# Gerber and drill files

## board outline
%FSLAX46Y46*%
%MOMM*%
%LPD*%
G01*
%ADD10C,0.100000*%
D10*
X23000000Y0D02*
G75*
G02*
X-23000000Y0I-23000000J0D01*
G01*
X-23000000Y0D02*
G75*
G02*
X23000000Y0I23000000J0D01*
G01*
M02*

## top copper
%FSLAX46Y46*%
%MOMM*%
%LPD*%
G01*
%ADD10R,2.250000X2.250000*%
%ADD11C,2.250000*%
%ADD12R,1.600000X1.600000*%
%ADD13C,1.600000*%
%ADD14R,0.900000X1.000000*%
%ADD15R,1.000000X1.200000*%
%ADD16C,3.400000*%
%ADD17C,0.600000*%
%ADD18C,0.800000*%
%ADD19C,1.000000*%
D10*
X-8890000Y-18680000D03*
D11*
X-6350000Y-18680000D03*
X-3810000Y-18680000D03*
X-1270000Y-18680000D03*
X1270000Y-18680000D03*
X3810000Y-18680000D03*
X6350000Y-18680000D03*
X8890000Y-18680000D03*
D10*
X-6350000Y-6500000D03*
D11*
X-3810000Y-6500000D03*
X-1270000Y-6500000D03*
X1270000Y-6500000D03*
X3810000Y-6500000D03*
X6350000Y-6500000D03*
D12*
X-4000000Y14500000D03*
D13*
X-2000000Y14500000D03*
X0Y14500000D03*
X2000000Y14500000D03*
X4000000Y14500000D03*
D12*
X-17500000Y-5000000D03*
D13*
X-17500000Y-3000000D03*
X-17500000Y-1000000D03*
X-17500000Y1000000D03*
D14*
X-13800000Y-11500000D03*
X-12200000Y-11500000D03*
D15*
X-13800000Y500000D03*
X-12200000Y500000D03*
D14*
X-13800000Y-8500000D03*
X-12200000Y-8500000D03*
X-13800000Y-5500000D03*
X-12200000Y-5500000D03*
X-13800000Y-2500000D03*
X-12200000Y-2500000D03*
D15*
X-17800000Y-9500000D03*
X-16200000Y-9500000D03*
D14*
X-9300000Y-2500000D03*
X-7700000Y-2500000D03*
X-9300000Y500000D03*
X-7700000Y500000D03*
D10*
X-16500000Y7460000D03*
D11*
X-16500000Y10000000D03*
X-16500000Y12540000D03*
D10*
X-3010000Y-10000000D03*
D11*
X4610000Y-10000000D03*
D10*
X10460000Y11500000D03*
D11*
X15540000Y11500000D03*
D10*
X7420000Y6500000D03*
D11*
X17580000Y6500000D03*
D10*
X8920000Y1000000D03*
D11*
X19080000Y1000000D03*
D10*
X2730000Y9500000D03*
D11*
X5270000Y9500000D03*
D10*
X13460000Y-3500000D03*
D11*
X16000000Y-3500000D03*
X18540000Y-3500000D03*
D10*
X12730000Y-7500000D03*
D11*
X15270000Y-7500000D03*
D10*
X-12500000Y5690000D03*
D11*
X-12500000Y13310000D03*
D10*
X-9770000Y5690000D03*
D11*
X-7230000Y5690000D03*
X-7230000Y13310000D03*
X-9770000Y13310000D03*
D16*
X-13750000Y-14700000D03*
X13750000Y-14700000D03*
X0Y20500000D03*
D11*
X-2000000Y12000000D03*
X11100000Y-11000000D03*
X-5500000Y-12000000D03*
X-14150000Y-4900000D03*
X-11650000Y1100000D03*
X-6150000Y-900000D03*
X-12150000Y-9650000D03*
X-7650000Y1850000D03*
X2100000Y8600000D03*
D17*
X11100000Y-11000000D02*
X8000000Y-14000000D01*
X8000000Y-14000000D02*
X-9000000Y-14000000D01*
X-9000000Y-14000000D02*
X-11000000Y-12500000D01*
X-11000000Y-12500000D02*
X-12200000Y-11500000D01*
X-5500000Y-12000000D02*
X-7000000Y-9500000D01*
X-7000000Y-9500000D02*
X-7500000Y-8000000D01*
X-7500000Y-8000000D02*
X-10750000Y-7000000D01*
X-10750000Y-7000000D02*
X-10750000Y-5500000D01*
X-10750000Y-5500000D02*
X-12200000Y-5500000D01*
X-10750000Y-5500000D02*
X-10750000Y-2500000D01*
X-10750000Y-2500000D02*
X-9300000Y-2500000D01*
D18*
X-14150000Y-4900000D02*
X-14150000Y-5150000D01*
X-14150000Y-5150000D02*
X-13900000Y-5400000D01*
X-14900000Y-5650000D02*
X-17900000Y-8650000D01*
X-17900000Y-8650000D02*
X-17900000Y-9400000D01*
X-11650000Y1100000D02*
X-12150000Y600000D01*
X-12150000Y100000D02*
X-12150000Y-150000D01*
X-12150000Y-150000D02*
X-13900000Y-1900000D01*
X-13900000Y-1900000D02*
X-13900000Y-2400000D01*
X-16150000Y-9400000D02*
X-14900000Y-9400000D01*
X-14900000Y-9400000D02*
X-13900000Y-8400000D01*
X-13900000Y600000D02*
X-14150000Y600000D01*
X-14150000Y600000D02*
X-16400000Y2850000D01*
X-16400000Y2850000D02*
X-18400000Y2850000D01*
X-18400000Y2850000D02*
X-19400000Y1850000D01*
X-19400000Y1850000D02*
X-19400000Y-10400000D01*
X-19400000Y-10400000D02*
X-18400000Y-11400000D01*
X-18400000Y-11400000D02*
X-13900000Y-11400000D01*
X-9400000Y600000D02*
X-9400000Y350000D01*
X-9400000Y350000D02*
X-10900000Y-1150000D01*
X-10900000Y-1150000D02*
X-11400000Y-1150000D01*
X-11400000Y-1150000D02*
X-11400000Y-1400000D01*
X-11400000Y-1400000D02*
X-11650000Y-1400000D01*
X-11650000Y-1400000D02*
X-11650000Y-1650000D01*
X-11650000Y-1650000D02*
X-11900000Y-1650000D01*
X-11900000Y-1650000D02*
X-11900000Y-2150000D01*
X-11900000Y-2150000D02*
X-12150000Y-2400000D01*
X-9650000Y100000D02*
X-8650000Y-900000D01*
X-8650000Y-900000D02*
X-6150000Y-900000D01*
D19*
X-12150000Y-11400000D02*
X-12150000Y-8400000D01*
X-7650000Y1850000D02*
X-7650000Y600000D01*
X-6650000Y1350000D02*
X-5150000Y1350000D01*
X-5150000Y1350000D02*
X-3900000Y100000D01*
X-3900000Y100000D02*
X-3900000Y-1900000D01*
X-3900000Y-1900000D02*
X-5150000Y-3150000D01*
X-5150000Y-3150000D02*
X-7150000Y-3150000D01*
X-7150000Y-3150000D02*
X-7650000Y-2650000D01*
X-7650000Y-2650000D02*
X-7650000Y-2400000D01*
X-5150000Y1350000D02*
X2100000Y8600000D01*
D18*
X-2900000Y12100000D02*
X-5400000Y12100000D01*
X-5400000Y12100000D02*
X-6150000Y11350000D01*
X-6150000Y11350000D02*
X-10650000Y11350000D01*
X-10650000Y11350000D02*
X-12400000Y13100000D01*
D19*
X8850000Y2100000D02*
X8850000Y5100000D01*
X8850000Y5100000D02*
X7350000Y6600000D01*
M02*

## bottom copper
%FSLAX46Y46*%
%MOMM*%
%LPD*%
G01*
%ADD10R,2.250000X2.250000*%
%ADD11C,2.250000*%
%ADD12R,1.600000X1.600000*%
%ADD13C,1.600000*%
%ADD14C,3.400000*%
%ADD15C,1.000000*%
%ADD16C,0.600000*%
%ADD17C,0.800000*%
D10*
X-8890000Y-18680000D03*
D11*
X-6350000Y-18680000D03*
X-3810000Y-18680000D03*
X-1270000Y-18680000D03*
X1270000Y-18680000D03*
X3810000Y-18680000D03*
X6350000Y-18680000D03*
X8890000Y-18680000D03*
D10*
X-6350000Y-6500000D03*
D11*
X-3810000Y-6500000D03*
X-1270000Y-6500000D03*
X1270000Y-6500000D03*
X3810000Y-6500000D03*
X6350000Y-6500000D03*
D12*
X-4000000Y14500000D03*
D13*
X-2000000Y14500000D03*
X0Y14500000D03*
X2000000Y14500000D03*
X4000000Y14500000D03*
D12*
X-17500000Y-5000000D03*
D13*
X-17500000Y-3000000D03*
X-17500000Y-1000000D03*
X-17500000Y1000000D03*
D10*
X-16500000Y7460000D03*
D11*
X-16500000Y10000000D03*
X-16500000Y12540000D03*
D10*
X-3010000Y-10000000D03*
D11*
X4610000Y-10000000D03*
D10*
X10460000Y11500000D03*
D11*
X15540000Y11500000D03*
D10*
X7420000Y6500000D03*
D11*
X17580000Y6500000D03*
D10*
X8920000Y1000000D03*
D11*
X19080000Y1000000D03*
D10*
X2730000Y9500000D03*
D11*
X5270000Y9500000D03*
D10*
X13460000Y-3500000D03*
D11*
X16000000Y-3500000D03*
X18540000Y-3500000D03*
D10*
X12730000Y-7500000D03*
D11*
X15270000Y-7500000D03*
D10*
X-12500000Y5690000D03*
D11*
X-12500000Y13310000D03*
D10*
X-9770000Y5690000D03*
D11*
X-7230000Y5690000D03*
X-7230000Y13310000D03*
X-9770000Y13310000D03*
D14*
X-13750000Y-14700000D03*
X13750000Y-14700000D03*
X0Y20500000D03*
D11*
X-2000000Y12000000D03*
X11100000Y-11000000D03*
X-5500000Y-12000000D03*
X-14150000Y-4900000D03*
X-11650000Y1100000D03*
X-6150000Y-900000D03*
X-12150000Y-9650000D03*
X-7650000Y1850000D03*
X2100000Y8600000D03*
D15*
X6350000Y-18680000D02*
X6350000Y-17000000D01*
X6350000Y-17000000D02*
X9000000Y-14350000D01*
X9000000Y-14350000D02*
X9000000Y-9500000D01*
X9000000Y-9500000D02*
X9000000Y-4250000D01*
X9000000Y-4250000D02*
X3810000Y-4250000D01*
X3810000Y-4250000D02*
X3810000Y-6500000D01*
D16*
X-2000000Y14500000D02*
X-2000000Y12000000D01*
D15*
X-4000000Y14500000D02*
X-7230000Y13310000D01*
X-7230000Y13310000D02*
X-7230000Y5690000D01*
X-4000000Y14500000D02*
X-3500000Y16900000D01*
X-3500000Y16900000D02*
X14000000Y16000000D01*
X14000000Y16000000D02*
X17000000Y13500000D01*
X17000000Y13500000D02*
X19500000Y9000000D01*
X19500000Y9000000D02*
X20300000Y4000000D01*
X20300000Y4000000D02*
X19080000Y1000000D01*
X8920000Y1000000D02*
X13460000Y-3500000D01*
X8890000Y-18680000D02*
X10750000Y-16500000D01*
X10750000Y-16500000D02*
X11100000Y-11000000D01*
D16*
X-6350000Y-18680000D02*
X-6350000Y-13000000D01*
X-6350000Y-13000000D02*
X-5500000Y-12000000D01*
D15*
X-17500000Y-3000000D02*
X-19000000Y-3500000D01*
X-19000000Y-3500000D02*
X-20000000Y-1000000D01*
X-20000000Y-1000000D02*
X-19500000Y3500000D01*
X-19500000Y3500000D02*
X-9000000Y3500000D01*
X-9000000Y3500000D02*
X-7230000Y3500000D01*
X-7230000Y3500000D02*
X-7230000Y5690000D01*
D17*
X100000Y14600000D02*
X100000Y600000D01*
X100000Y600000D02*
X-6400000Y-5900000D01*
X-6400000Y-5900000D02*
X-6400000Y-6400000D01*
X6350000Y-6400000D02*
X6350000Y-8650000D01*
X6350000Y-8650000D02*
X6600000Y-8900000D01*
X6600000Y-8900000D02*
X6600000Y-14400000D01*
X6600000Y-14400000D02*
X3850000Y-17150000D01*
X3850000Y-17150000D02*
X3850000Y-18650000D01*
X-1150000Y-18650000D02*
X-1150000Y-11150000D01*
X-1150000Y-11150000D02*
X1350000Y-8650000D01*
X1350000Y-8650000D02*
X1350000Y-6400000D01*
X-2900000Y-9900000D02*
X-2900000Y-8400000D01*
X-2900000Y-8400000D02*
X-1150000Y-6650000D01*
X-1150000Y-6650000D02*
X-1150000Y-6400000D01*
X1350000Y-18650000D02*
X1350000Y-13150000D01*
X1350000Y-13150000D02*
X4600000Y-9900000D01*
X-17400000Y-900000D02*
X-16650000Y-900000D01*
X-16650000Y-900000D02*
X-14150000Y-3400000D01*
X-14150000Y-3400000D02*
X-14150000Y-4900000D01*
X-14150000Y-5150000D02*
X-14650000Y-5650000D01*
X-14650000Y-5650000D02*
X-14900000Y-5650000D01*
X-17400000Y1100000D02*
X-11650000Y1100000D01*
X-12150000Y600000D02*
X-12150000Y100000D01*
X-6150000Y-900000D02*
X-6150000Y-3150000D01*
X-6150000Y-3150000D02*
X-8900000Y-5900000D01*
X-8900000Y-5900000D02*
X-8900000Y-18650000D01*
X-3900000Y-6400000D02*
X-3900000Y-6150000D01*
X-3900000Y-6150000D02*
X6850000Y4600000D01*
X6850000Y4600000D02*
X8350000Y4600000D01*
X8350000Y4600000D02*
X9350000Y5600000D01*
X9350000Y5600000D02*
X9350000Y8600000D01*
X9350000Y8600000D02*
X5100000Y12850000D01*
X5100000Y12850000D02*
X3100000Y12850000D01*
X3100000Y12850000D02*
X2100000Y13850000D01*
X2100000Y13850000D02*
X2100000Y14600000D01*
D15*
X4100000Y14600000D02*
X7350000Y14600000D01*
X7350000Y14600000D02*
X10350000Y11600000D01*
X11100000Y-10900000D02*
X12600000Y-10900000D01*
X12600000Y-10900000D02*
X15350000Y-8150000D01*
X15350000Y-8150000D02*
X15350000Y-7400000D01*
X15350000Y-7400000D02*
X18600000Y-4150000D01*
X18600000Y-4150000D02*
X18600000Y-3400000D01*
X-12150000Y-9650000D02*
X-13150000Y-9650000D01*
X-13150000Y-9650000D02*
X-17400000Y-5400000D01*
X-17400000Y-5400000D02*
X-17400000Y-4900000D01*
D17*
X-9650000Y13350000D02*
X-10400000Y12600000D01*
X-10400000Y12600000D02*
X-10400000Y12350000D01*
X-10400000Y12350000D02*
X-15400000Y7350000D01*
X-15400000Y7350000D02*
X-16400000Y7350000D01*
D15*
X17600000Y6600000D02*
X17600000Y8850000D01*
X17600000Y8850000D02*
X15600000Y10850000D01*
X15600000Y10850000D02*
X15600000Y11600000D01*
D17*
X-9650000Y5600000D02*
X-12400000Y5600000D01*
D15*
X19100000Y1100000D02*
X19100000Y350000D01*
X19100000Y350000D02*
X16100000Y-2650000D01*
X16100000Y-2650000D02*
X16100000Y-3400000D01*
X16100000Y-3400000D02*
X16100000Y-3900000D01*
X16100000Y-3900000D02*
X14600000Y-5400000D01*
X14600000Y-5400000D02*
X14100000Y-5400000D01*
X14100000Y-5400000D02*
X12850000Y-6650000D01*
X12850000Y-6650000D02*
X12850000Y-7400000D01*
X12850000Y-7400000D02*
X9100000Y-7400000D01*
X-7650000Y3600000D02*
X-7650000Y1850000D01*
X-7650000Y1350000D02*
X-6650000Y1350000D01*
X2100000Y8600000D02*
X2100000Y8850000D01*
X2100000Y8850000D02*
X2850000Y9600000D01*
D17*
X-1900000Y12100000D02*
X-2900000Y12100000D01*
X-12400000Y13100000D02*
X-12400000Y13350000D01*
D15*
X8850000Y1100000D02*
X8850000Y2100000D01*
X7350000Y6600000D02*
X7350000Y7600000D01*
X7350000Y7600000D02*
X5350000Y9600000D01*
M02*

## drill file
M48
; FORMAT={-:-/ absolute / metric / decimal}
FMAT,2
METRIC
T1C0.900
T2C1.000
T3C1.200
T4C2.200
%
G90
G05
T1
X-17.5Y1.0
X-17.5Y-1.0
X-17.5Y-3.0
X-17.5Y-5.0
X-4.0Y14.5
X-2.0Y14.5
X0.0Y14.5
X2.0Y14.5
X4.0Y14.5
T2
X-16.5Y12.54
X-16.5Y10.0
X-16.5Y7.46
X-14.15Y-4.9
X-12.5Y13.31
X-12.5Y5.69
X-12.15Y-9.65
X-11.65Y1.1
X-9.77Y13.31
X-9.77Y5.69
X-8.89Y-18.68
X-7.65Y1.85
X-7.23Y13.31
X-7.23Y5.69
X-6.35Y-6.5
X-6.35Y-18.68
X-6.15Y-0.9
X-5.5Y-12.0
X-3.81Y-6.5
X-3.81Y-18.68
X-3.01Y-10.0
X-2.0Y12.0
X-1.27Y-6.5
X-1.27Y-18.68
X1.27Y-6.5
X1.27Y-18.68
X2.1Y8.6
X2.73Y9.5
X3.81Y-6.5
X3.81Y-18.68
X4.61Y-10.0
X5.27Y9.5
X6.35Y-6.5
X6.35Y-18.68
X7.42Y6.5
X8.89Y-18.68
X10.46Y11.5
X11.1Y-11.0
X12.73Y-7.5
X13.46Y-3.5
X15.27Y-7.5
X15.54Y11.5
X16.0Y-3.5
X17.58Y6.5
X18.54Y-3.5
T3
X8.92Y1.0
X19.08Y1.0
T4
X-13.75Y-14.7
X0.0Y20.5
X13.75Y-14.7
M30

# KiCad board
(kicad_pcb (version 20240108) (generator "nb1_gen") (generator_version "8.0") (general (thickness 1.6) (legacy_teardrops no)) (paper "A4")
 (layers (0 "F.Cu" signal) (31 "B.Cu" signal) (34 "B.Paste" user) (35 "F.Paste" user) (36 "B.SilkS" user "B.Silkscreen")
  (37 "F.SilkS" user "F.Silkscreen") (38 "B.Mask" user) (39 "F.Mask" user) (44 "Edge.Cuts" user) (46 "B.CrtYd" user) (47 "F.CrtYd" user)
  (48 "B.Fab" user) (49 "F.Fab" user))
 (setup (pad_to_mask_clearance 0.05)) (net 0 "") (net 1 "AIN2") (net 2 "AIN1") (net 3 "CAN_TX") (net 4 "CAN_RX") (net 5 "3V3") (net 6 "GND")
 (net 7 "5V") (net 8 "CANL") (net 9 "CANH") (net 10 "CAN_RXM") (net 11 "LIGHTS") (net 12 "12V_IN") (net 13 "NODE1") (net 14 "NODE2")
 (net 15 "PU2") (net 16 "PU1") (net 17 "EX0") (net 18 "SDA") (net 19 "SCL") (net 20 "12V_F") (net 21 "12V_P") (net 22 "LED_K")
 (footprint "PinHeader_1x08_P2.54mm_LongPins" (layer "F.Cu") (at 0 18.68 0)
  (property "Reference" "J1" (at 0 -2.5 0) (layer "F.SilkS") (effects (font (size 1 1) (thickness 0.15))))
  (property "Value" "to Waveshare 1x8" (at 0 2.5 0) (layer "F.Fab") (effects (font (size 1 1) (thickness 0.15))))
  (pad "1" thru_hole rect (at -8.89 0 0) (size 2.25 2.25) (drill 1.0) (layers "*.Cu" "*.Mask") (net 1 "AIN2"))
  (pad "2" thru_hole circle (at -6.35 0 0) (size 2.25 2.25) (drill 1.0) (layers "*.Cu" "*.Mask") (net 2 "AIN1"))
  (pad "3" thru_hole circle (at -3.81 0 0) (size 2.25 2.25) (drill 1.0) (layers "*.Cu" "*.Mask"))
  (pad "4" thru_hole circle (at -1.27 0 0) (size 2.25 2.25) (drill 1.0) (layers "*.Cu" "*.Mask") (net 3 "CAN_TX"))
  (pad "5" thru_hole circle (at 1.27 0 0) (size 2.25 2.25) (drill 1.0) (layers "*.Cu" "*.Mask") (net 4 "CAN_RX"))
  (pad "6" thru_hole circle (at 3.81 0 0) (size 2.25 2.25) (drill 1.0) (layers "*.Cu" "*.Mask") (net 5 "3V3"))
  (pad "7" thru_hole circle (at 6.35 0 0) (size 2.25 2.25) (drill 1.0) (layers "*.Cu" "*.Mask") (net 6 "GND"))
  (pad "8" thru_hole circle (at 8.89 0 0) (size 2.25 2.25) (drill 1.0) (layers "*.Cu" "*.Mask") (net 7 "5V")))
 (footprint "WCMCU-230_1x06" (layer "F.Cu") (at 0 6.5 0)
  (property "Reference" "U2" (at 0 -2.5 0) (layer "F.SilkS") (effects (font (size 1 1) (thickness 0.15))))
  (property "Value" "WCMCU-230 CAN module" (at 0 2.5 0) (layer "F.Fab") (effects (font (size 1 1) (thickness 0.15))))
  (pad "1" thru_hole rect (at -6.35 0 0) (size 2.25 2.25) (drill 1.0) (layers "*.Cu" "*.Mask") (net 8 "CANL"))
  (pad "2" thru_hole circle (at -3.81 0 0) (size 2.25 2.25) (drill 1.0) (layers "*.Cu" "*.Mask") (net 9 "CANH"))
  (pad "3" thru_hole circle (at -1.27 0 0) (size 2.25 2.25) (drill 1.0) (layers "*.Cu" "*.Mask") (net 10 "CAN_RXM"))
  (pad "4" thru_hole circle (at 1.27 0 0) (size 2.25 2.25) (drill 1.0) (layers "*.Cu" "*.Mask") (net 3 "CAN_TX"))
  (pad "5" thru_hole circle (at 3.81 0 0) (size 2.25 2.25) (drill 1.0) (layers "*.Cu" "*.Mask") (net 6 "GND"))
  (pad "6" thru_hole circle (at 6.35 0 0) (size 2.25 2.25) (drill 1.0) (layers "*.Cu" "*.Mask") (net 5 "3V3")))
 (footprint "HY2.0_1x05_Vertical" (layer "F.Cu") (at 0 -14.5 0)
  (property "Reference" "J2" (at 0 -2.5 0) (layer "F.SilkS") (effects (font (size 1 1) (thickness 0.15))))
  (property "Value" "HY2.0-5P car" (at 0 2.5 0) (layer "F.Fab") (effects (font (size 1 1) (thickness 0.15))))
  (pad "1" thru_hole rect (at -4.0 0 0) (size 1.6 1.6) (drill 0.9) (layers "*.Cu" "*.Mask") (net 6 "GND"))
  (pad "2" thru_hole circle (at -2.0 0 0) (size 1.6 1.6) (drill 0.9) (layers "*.Cu" "*.Mask") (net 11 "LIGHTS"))
  (pad "3" thru_hole circle (at 0.0 0 0) (size 1.6 1.6) (drill 0.9) (layers "*.Cu" "*.Mask") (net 8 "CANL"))
  (pad "4" thru_hole circle (at 2.0 0 0) (size 1.6 1.6) (drill 0.9) (layers "*.Cu" "*.Mask") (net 9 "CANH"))
  (pad "5" thru_hole circle (at 4.0 0 0) (size 1.6 1.6) (drill 0.9) (layers "*.Cu" "*.Mask") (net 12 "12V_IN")))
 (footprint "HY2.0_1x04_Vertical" (layer "F.Cu") (at -17.5 2.0 0)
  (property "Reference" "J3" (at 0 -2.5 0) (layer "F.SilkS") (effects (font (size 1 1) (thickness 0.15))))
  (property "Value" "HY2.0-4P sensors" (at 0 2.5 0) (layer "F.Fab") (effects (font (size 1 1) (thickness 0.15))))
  (pad "1" thru_hole rect (at 0 3.0 0) (size 1.6 1.6) (drill 0.9) (layers "*.Cu" "*.Mask") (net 7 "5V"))
  (pad "2" thru_hole circle (at 0 1.0 0) (size 1.6 1.6) (drill 0.9) (layers "*.Cu" "*.Mask") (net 6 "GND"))
  (pad "3" thru_hole circle (at 0 -1.0 0) (size 1.6 1.6) (drill 0.9) (layers "*.Cu" "*.Mask") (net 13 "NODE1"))
  (pad "4" thru_hole circle (at 0 -3.0 0) (size 1.6 1.6) (drill 0.9) (layers "*.Cu" "*.Mask") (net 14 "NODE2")))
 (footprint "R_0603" (layer "F.Cu") (at -13.0 11.5 0)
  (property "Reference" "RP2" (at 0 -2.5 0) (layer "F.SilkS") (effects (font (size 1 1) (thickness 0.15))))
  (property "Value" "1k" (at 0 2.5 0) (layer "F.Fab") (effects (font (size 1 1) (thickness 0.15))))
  (pad "1" smd rect (at -0.8 0 0) (size 0.9 1.0) (layers "F.Cu" "F.Mask") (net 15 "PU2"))
  (pad "2" smd rect (at 0.8 0 0) (size 0.9 1.0) (layers "F.Cu" "F.Mask") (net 7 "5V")))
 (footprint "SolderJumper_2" (layer "F.Cu") (at -13.0 -0.5 0)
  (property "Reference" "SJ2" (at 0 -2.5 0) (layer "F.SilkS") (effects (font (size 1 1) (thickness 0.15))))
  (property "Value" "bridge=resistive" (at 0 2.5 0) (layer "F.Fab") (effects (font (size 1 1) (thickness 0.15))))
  (pad "1" smd rect (at -0.8 0 0) (size 1.0 1.2) (layers "F.Cu" "F.Mask") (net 15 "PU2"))
  (pad "2" smd rect (at 0.8 0 0) (size 1.0 1.2) (layers "F.Cu" "F.Mask") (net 14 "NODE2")))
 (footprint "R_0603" (layer "F.Cu") (at -13.0 8.5 0)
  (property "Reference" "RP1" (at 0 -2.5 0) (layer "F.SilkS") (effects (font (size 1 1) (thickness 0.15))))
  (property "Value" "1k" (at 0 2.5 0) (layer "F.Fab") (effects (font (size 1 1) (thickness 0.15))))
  (pad "1" smd rect (at -0.8 0 0) (size 0.9 1.0) (layers "F.Cu" "F.Mask") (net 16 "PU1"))
  (pad "2" smd rect (at 0.8 0 0) (size 0.9 1.0) (layers "F.Cu" "F.Mask") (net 7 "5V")))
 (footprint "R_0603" (layer "F.Cu") (at -13.0 5.5 0)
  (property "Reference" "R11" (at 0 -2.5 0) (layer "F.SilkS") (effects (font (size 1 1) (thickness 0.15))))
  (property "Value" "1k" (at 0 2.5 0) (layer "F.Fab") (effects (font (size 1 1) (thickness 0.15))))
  (pad "1" smd rect (at -0.8 0 0) (size 0.9 1.0) (layers "F.Cu" "F.Mask") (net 13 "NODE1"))
  (pad "2" smd rect (at 0.8 0 0) (size 0.9 1.0) (layers "F.Cu" "F.Mask") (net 2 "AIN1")))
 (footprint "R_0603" (layer "F.Cu") (at -13.0 2.5 0)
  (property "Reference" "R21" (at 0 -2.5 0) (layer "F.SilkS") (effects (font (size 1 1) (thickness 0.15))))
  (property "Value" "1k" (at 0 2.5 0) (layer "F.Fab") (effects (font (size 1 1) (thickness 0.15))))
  (pad "1" smd rect (at -0.8 0 0) (size 0.9 1.0) (layers "F.Cu" "F.Mask") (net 14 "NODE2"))
  (pad "2" smd rect (at 0.8 0 0) (size 0.9 1.0) (layers "F.Cu" "F.Mask") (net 1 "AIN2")))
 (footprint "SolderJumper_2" (layer "F.Cu") (at -17.0 9.5 0)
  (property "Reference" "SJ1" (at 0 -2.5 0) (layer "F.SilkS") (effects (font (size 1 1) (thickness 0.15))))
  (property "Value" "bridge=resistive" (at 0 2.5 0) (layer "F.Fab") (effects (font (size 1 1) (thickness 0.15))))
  (pad "1" smd rect (at -0.8 0 0) (size 1.0 1.2) (layers "F.Cu" "F.Mask") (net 13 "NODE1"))
  (pad "2" smd rect (at 0.8 0 0) (size 1.0 1.2) (layers "F.Cu" "F.Mask") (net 16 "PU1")))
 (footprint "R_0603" (layer "F.Cu") (at -8.5 2.5 0)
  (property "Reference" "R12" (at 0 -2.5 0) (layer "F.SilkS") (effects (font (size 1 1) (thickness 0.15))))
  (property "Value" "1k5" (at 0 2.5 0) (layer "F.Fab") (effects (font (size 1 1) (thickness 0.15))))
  (pad "1" smd rect (at -0.8 0 0) (size 0.9 1.0) (layers "F.Cu" "F.Mask") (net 2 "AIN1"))
  (pad "2" smd rect (at 0.8 0 0) (size 0.9 1.0) (layers "F.Cu" "F.Mask") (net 6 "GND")))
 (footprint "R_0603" (layer "F.Cu") (at -8.5 -0.5 0)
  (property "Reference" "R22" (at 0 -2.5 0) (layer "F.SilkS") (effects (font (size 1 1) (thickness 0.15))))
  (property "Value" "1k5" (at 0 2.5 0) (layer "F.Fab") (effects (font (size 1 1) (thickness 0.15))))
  (pad "1" smd rect (at -0.8 0 0) (size 0.9 1.0) (layers "F.Cu" "F.Mask") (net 1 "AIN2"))
  (pad "2" smd rect (at 0.8 0 0) (size 0.9 1.0) (layers "F.Cu" "F.Mask") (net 6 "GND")))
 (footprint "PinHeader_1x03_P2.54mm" (layer "F.Cu") (at -16.5 -10.0 0)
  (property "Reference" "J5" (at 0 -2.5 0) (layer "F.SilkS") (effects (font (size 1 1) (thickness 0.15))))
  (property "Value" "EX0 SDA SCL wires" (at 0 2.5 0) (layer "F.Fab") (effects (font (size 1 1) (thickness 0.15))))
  (pad "1" thru_hole rect (at 0 2.54 0) (size 2.25 2.25) (drill 1.0) (layers "*.Cu" "*.Mask") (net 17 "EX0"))
  (pad "2" thru_hole circle (at 0 -0.0 0) (size 2.25 2.25) (drill 1.0) (layers "*.Cu" "*.Mask") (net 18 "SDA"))
  (pad "3" thru_hole circle (at 0 -2.54 0) (size 2.25 2.25) (drill 1.0) (layers "*.Cu" "*.Mask") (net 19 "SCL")))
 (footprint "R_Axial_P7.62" (layer "F.Cu") (at 0.8 10.0 0)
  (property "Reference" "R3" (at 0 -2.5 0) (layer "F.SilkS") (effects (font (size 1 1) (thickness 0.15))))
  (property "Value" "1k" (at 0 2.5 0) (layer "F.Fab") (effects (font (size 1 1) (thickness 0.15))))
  (pad "1" thru_hole rect (at -3.81 0 0) (size 2.25 2.25) (drill 1.0) (layers "*.Cu" "*.Mask") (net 10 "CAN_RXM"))
  (pad "2" thru_hole circle (at 3.81 0 0) (size 2.25 2.25) (drill 1.0) (layers "*.Cu" "*.Mask") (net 4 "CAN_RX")))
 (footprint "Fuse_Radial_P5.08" (layer "F.Cu") (at 13.0 -11.5 0)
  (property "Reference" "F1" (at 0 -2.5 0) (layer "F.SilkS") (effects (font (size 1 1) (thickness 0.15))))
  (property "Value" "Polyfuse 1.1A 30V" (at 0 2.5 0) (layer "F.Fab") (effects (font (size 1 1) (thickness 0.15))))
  (pad "1" thru_hole rect (at -2.54 0 0) (size 2.25 2.25) (drill 1.0) (layers "*.Cu" "*.Mask") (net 12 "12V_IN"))
  (pad "2" thru_hole circle (at 2.54 0 0) (size 2.25 2.25) (drill 1.0) (layers "*.Cu" "*.Mask") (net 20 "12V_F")))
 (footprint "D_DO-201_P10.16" (layer "F.Cu") (at 12.5 -6.5 0)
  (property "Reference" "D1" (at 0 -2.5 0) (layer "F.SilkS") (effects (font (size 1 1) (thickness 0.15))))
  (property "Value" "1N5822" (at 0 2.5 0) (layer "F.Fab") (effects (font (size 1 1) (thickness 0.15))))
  (pad "1" thru_hole rect (at -5.08 0 0) (size 2.25 2.25) (drill 1.0) (layers "*.Cu" "*.Mask") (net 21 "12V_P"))
  (pad "2" thru_hole circle (at 5.08 0 0) (size 2.25 2.25) (drill 1.0) (layers "*.Cu" "*.Mask") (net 20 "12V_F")))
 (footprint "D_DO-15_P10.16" (layer "F.Cu") (at 14.0 -1.0 0)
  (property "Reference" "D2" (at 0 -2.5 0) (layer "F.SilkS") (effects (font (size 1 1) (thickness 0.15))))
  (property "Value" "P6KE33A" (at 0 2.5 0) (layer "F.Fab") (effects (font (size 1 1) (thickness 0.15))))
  (pad "1" thru_hole rect (at -5.08 0 0) (size 2.25 2.25) (drill 1.2) (layers "*.Cu" "*.Mask") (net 21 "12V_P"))
  (pad "2" thru_hole circle (at 5.08 0 0) (size 2.25 2.25) (drill 1.2) (layers "*.Cu" "*.Mask") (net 6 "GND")))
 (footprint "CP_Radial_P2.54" (layer "F.Cu") (at 4.0 -9.5 0)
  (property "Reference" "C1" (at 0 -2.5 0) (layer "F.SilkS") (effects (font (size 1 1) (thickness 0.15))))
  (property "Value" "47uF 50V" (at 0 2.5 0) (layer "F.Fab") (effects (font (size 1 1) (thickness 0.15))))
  (pad "1" thru_hole rect (at -1.27 0 0) (size 2.25 2.25) (drill 1.0) (layers "*.Cu" "*.Mask") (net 6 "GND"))
  (pad "2" thru_hole circle (at 1.27 0 0) (size 2.25 2.25) (drill 1.0) (layers "*.Cu" "*.Mask") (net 21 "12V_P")))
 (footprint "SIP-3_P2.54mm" (layer "F.Cu") (at 16.0 3.5 0)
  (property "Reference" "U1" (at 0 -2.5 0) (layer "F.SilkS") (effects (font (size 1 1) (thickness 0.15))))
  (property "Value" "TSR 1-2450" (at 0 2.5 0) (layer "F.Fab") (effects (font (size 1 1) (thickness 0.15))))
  (pad "1" thru_hole rect (at -2.54 0 0) (size 2.25 2.25) (drill 1.0) (layers "*.Cu" "*.Mask") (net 21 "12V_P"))
  (pad "2" thru_hole circle (at 0.0 0 0) (size 2.25 2.25) (drill 1.0) (layers "*.Cu" "*.Mask") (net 6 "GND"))
  (pad "3" thru_hole circle (at 2.54 0 0) (size 2.25 2.25) (drill 1.0) (layers "*.Cu" "*.Mask") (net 7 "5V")))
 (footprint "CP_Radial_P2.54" (layer "F.Cu") (at 14.0 7.5 0)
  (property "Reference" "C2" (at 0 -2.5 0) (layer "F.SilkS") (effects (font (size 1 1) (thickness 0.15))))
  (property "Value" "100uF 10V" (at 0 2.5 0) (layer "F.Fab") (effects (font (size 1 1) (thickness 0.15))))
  (pad "1" thru_hole rect (at -1.27 0 0) (size 2.25 2.25) (drill 1.0) (layers "*.Cu" "*.Mask") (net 6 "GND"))
  (pad "2" thru_hole circle (at 1.27 0 0) (size 2.25 2.25) (drill 1.0) (layers "*.Cu" "*.Mask") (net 7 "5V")))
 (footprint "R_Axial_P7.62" (layer "F.Cu") (at -12.5 -9.5 90)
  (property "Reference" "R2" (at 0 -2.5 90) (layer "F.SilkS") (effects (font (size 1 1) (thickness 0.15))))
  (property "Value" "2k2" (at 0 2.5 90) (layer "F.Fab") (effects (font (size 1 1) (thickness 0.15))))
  (pad "1" thru_hole rect (at -3.81 0 90) (size 2.25 2.25) (drill 1.0) (layers "*.Cu" "*.Mask") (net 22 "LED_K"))
  (pad "2" thru_hole circle (at 3.81 0 90) (size 2.25 2.25) (drill 1.0) (layers "*.Cu" "*.Mask") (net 11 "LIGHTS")))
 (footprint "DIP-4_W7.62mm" (layer "F.Cu") (at -8.5 -9.5 0)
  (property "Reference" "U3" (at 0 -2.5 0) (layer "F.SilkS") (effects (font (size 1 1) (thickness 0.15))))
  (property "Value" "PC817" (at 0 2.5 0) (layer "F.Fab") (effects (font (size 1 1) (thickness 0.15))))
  (pad "1" thru_hole rect (at -1.27 3.81 0) (size 2.25 2.25) (drill 1.0) (layers "*.Cu" "*.Mask") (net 22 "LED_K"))
  (pad "2" thru_hole circle (at 1.27 3.81 0) (size 2.25 2.25) (drill 1.0) (layers "*.Cu" "*.Mask") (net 6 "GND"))
  (pad "3" thru_hole circle (at 1.27 -3.81 0) (size 2.25 2.25) (drill 1.0) (layers "*.Cu" "*.Mask") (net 6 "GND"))
  (pad "4" thru_hole circle (at -1.27 -3.81 0) (size 2.25 2.25) (drill 1.0) (layers "*.Cu" "*.Mask") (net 17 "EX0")))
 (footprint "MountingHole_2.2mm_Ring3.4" (layer "F.Cu") (at -13.75 14.7 0)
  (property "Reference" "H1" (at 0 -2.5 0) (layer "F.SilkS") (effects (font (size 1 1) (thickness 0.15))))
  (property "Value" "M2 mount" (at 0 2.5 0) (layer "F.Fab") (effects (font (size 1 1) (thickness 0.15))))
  (pad "1" thru_hole circle (at 0 0 0) (size 3.4 3.4) (drill 2.2) (layers "*.Cu" "*.Mask")))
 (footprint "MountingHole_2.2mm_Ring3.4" (layer "F.Cu") (at 13.75 14.7 0)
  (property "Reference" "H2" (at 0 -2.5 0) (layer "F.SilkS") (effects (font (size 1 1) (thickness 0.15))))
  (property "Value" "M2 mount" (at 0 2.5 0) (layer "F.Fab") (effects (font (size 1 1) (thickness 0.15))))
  (pad "1" thru_hole circle (at 0 0 0) (size 3.4 3.4) (drill 2.2) (layers "*.Cu" "*.Mask")))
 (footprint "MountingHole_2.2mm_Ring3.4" (layer "F.Cu") (at 0 -20.5 0)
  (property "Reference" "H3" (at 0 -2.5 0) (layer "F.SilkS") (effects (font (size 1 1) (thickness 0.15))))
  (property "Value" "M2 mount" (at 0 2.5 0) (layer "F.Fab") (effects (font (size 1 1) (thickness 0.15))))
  (pad "1" thru_hole circle (at 0 0 0) (size 3.4 3.4) (drill 2.2) (layers "*.Cu" "*.Mask")))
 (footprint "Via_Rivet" (layer "F.Cu") (at -2.0 -12.0 0)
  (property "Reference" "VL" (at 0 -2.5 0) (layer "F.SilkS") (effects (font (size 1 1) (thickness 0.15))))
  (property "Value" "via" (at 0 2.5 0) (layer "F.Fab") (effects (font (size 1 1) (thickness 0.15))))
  (pad "1" thru_hole circle (at 0 0 0) (size 2.25 2.25) (drill 1.0) (layers "*.Cu" "*.Mask") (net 11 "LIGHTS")))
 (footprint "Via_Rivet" (layer "F.Cu") (at 11.1 11.0 0)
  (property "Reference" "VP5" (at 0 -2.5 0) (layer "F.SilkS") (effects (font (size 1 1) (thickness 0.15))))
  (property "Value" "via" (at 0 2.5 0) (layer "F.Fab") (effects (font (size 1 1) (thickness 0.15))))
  (pad "1" thru_hole circle (at 0 0 0) (size 2.25 2.25) (drill 1.0) (layers "*.Cu" "*.Mask") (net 7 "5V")))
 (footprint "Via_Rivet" (layer "F.Cu") (at -5.5 12.0 0)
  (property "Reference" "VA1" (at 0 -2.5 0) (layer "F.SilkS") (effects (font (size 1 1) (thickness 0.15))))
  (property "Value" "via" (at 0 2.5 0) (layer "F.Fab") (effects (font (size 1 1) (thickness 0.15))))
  (pad "1" thru_hole circle (at 0 0 0) (size 2.25 2.25) (drill 1.0) (layers "*.Cu" "*.Mask") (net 2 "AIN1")))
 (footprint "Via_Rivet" (layer "F.Cu") (at -14.15 4.9 0)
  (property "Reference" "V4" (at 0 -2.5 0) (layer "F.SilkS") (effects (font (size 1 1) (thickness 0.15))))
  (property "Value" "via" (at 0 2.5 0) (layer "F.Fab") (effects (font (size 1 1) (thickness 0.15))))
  (pad "1" thru_hole circle (at 0 0 0) (size 2.25 2.25) (drill 1.0) (layers "*.Cu" "*.Mask") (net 13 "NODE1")))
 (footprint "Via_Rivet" (layer "F.Cu") (at -11.65 -1.1 0)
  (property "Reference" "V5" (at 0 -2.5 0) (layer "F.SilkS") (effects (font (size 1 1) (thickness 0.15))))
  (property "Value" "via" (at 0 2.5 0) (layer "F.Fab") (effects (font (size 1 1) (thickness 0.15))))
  (pad "1" thru_hole circle (at 0 0 0) (size 2.25 2.25) (drill 1.0) (layers "*.Cu" "*.Mask") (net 14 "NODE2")))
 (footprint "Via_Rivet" (layer "F.Cu") (at -6.15 0.9 0)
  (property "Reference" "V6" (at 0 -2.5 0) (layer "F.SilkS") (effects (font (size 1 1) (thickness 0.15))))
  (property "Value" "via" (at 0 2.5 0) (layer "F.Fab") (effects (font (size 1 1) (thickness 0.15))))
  (pad "1" thru_hole circle (at 0 0 0) (size 2.25 2.25) (drill 1.0) (layers "*.Cu" "*.Mask") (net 1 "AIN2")))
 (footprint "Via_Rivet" (layer "F.Cu") (at -12.15 9.65 0)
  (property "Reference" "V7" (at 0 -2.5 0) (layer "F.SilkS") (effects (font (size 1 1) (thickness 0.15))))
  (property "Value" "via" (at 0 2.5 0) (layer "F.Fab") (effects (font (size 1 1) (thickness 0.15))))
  (pad "1" thru_hole circle (at 0 0 0) (size 2.25 2.25) (drill 1.0) (layers "*.Cu" "*.Mask") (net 7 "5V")))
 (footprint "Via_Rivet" (layer "F.Cu") (at -7.65 -1.85 0)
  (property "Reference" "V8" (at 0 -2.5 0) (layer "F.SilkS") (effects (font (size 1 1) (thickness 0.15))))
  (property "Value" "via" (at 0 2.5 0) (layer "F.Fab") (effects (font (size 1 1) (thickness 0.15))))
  (pad "1" thru_hole circle (at 0 0 0) (size 2.25 2.25) (drill 1.0) (layers "*.Cu" "*.Mask") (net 6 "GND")))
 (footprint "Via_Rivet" (layer "F.Cu") (at 2.1 -8.6 0)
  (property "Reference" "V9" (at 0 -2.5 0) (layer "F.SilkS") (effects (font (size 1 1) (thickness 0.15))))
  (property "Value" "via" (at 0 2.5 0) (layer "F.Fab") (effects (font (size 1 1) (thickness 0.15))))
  (pad "1" thru_hole circle (at 0 0 0) (size 2.25 2.25) (drill 1.0) (layers "*.Cu" "*.Mask") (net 6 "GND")))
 (gr_circle (center 0 0) (end 23.0 0) (stroke (width 0.1) (type default)) (fill none) (layer "Edge.Cuts"))
 (segment (start 6.35 18.68) (end 6.35 17.0) (width 1.0) (layer "B.Cu") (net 6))
 (segment (start 6.35 17.0) (end 9.0 14.35) (width 1.0) (layer "B.Cu") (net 6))
 (segment (start 9.0 14.35) (end 9.0 9.5) (width 1.0) (layer "B.Cu") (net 6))
 (segment (start 9.0 9.5) (end 9.0 4.25) (width 1.0) (layer "B.Cu") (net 6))
 (segment (start 9.0 4.25) (end 3.81 4.25) (width 1.0) (layer "B.Cu") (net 6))
 (segment (start 3.81 4.25) (end 3.81 6.5) (width 1.0) (layer "B.Cu") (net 6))
 (segment (start -2.0 -14.5) (end -2.0 -12.0) (width 0.6) (layer "B.Cu") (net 11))
 (segment (start -4.0 -14.5) (end -7.23 -13.31) (width 1.0) (layer "B.Cu") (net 6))
 (segment (start -7.23 -13.31) (end -7.23 -5.69) (width 1.0) (layer "B.Cu") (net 6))
 (segment (start -4.0 -14.5) (end -3.5 -16.9) (width 1.0) (layer "B.Cu") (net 6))
 (segment (start -3.5 -16.9) (end 14.0 -16.0) (width 1.0) (layer "B.Cu") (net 6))
 (segment (start 14.0 -16.0) (end 17.0 -13.5) (width 1.0) (layer "B.Cu") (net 6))
 (segment (start 17.0 -13.5) (end 19.5 -9.0) (width 1.0) (layer "B.Cu") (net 6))
 (segment (start 19.5 -9.0) (end 20.3 -4.0) (width 1.0) (layer "B.Cu") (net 6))
 (segment (start 20.3 -4.0) (end 19.08 -1.0) (width 1.0) (layer "B.Cu") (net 6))
 (segment (start 8.92 -1.0) (end 13.46 3.5) (width 1.0) (layer "B.Cu") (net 21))
 (segment (start 8.89 18.68) (end 10.75 16.5) (width 1.0) (layer "B.Cu") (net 7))
 (segment (start 10.75 16.5) (end 11.1 11.0) (width 1.0) (layer "B.Cu") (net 7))
 (segment (start 11.1 11.0) (end 8.0 14.0) (width 0.6) (layer "F.Cu") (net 7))
 (segment (start 8.0 14.0) (end -9.0 14.0) (width 0.6) (layer "F.Cu") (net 7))
 (segment (start -9.0 14.0) (end -11.0 12.5) (width 0.6) (layer "F.Cu") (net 7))
 (segment (start -11.0 12.5) (end -12.2 11.5) (width 0.6) (layer "F.Cu") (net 7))
 (segment (start -6.35 18.68) (end -6.35 13.0) (width 0.6) (layer "B.Cu") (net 2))
 (segment (start -6.35 13.0) (end -5.5 12.0) (width 0.6) (layer "B.Cu") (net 2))
 (segment (start -5.5 12.0) (end -7.0 9.5) (width 0.6) (layer "F.Cu") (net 2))
 (segment (start -7.0 9.5) (end -7.5 8.0) (width 0.6) (layer "F.Cu") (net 2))
 (segment (start -7.5 8.0) (end -10.75 7.0) (width 0.6) (layer "F.Cu") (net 2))
 (segment (start -10.75 7.0) (end -10.75 5.5) (width 0.6) (layer "F.Cu") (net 2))
 (segment (start -10.75 5.5) (end -12.2 5.5) (width 0.6) (layer "F.Cu") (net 2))
 (segment (start -10.75 5.5) (end -10.75 2.5) (width 0.6) (layer "F.Cu") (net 2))
 (segment (start -10.75 2.5) (end -9.3 2.5) (width 0.6) (layer "F.Cu") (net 2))
 (segment (start -17.5 3.0) (end -19.0 3.5) (width 1.0) (layer "B.Cu") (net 6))
 (segment (start -19.0 3.5) (end -20.0 1.0) (width 1.0) (layer "B.Cu") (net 6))
 (segment (start -20.0 1.0) (end -19.5 -3.5) (width 1.0) (layer "B.Cu") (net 6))
 (segment (start -19.5 -3.5) (end -9.0 -3.5) (width 1.0) (layer "B.Cu") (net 6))
 (segment (start -9.0 -3.5) (end -7.23 -3.5) (width 1.0) (layer "B.Cu") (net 6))
 (segment (start -7.23 -3.5) (end -7.23 -5.69) (width 1.0) (layer "B.Cu") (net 6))
 (segment (start 0.1 -14.6) (end 0.1 -0.6) (width 0.8) (layer "B.Cu") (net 8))
 (segment (start 0.1 -0.6) (end -6.4 5.9) (width 0.8) (layer "B.Cu") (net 8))
 (segment (start -6.4 5.9) (end -6.4 6.4) (width 0.8) (layer "B.Cu") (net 8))
 (segment (start 6.35 6.4) (end 6.35 8.65) (width 0.8) (layer "B.Cu") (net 5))
 (segment (start 6.35 8.65) (end 6.6 8.9) (width 0.8) (layer "B.Cu") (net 5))
 (segment (start 6.6 8.9) (end 6.6 14.4) (width 0.8) (layer "B.Cu") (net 5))
 (segment (start 6.6 14.4) (end 3.85 17.15) (width 0.8) (layer "B.Cu") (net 5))
 (segment (start 3.85 17.15) (end 3.85 18.65) (width 0.8) (layer "B.Cu") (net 5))
 (segment (start -1.15 18.65) (end -1.15 11.15) (width 0.8) (layer "B.Cu") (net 3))
 (segment (start -1.15 11.15) (end 1.35 8.65) (width 0.8) (layer "B.Cu") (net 3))
 (segment (start 1.35 8.65) (end 1.35 6.4) (width 0.8) (layer "B.Cu") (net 3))
 (segment (start -2.9 9.9) (end -2.9 8.4) (width 0.8) (layer "B.Cu") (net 10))
 (segment (start -2.9 8.4) (end -1.15 6.65) (width 0.8) (layer "B.Cu") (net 10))
 (segment (start -1.15 6.65) (end -1.15 6.4) (width 0.8) (layer "B.Cu") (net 10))
 (segment (start 1.35 18.65) (end 1.35 13.15) (width 0.8) (layer "B.Cu") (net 4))
 (segment (start 1.35 13.15) (end 4.6 9.9) (width 0.8) (layer "B.Cu") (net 4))
 (segment (start -17.4 0.9) (end -16.65 0.9) (width 0.8) (layer "B.Cu") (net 13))
 (segment (start -16.65 0.9) (end -14.15 3.4) (width 0.8) (layer "B.Cu") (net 13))
 (segment (start -14.15 3.4) (end -14.15 4.9) (width 0.8) (layer "B.Cu") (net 13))
 (segment (start -14.15 4.9) (end -14.15 5.15) (width 0.8) (layer "F.Cu") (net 13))
 (segment (start -14.15 5.15) (end -13.9 5.4) (width 0.8) (layer "F.Cu") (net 13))
 (segment (start -14.15 5.15) (end -14.65 5.65) (width 0.8) (layer "B.Cu") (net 13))
 (segment (start -14.65 5.65) (end -14.9 5.65) (width 0.8) (layer "B.Cu") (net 13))
 (segment (start -14.9 5.65) (end -17.9 8.65) (width 0.8) (layer "F.Cu") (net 13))
 (segment (start -17.9 8.65) (end -17.9 9.4) (width 0.8) (layer "F.Cu") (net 13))
 (segment (start -17.4 -1.1) (end -11.65 -1.1) (width 0.8) (layer "B.Cu") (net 14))
 (segment (start -11.65 -1.1) (end -12.15 -0.6) (width 0.8) (layer "F.Cu") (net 14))
 (segment (start -12.15 -0.6) (end -12.15 -0.1) (width 0.8) (layer "B.Cu") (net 14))
 (segment (start -12.15 -0.1) (end -12.15 0.15) (width 0.8) (layer "F.Cu") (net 14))
 (segment (start -12.15 0.15) (end -13.9 1.9) (width 0.8) (layer "F.Cu") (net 14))
 (segment (start -13.9 1.9) (end -13.9 2.4) (width 0.8) (layer "F.Cu") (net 14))
 (segment (start -16.15 9.4) (end -14.9 9.4) (width 0.8) (layer "F.Cu") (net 16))
 (segment (start -14.9 9.4) (end -13.9 8.4) (width 0.8) (layer "F.Cu") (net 16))
 (segment (start -13.9 -0.6) (end -14.15 -0.6) (width 0.8) (layer "F.Cu") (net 15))
 (segment (start -14.15 -0.6) (end -16.4 -2.85) (width 0.8) (layer "F.Cu") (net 15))
 (segment (start -16.4 -2.85) (end -18.4 -2.85) (width 0.8) (layer "F.Cu") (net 15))
 (segment (start -18.4 -2.85) (end -19.4 -1.85) (width 0.8) (layer "F.Cu") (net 15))
 (segment (start -19.4 -1.85) (end -19.4 10.4) (width 0.8) (layer "F.Cu") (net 15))
 (segment (start -19.4 10.4) (end -18.4 11.4) (width 0.8) (layer "F.Cu") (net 15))
 (segment (start -18.4 11.4) (end -13.9 11.4) (width 0.8) (layer "F.Cu") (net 15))
 (segment (start -9.4 -0.6) (end -9.4 -0.35) (width 0.8) (layer "F.Cu") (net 1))
 (segment (start -9.4 -0.35) (end -10.9 1.15) (width 0.8) (layer "F.Cu") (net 1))
 (segment (start -10.9 1.15) (end -11.4 1.15) (width 0.8) (layer "F.Cu") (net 1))
 (segment (start -11.4 1.15) (end -11.4 1.4) (width 0.8) (layer "F.Cu") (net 1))
 (segment (start -11.4 1.4) (end -11.65 1.4) (width 0.8) (layer "F.Cu") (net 1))
 (segment (start -11.65 1.4) (end -11.65 1.65) (width 0.8) (layer "F.Cu") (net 1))
 (segment (start -11.65 1.65) (end -11.9 1.65) (width 0.8) (layer "F.Cu") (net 1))
 (segment (start -11.9 1.65) (end -11.9 2.15) (width 0.8) (layer "F.Cu") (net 1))
 (segment (start -11.9 2.15) (end -12.15 2.4) (width 0.8) (layer "F.Cu") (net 1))
 (segment (start -9.65 -0.1) (end -8.65 0.9) (width 0.8) (layer "F.Cu") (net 1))
 (segment (start -8.65 0.9) (end -6.15 0.9) (width 0.8) (layer "F.Cu") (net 1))
 (segment (start -6.15 0.9) (end -6.15 3.15) (width 0.8) (layer "B.Cu") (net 1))
 (segment (start -6.15 3.15) (end -8.9 5.9) (width 0.8) (layer "B.Cu") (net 1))
 (segment (start -8.9 5.9) (end -8.9 18.65) (width 0.8) (layer "B.Cu") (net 1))
 (segment (start -3.9 6.4) (end -3.9 6.15) (width 0.8) (layer "B.Cu") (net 9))
 (segment (start -3.9 6.15) (end 6.85 -4.6) (width 0.8) (layer "B.Cu") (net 9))
 (segment (start 6.85 -4.6) (end 8.35 -4.6) (width 0.8) (layer "B.Cu") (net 9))
 (segment (start 8.35 -4.6) (end 9.35 -5.6) (width 0.8) (layer "B.Cu") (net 9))
 (segment (start 9.35 -5.6) (end 9.35 -8.6) (width 0.8) (layer "B.Cu") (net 9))
 (segment (start 9.35 -8.6) (end 5.1 -12.85) (width 0.8) (layer "B.Cu") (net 9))
 (segment (start 5.1 -12.85) (end 3.1 -12.85) (width 0.8) (layer "B.Cu") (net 9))
 (segment (start 3.1 -12.85) (end 2.1 -13.85) (width 0.8) (layer "B.Cu") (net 9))
 (segment (start 2.1 -13.85) (end 2.1 -14.6) (width 0.8) (layer "B.Cu") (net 9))
 (segment (start 4.1 -14.6) (end 7.35 -14.6) (width 1.0) (layer "B.Cu") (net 12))
 (segment (start 7.35 -14.6) (end 10.35 -11.6) (width 1.0) (layer "B.Cu") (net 12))
 (segment (start -12.15 11.4) (end -12.15 8.4) (width 1.0) (layer "F.Cu") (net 7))
 (segment (start 11.1 10.9) (end 12.6 10.9) (width 1.0) (layer "B.Cu") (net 7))
 (segment (start 12.6 10.9) (end 15.35 8.15) (width 1.0) (layer "B.Cu") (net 7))
 (segment (start 15.35 8.15) (end 15.35 7.4) (width 1.0) (layer "B.Cu") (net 7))
 (segment (start 15.35 7.4) (end 18.6 4.15) (width 1.0) (layer "B.Cu") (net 7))
 (segment (start 18.6 4.15) (end 18.6 3.4) (width 1.0) (layer "B.Cu") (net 7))
 (segment (start -12.15 9.65) (end -13.15 9.65) (width 1.0) (layer "B.Cu") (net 7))
 (segment (start -13.15 9.65) (end -17.4 5.4) (width 1.0) (layer "B.Cu") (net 7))
 (segment (start -17.4 5.4) (end -17.4 4.9) (width 1.0) (layer "B.Cu") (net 7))
 (segment (start -9.65 -13.35) (end -10.4 -12.6) (width 0.8) (layer "B.Cu") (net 17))
 (segment (start -10.4 -12.6) (end -10.4 -12.35) (width 0.8) (layer "B.Cu") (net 17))
 (segment (start -10.4 -12.35) (end -15.4 -7.35) (width 0.8) (layer "B.Cu") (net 17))
 (segment (start -15.4 -7.35) (end -16.4 -7.35) (width 0.8) (layer "B.Cu") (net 17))
 (segment (start 17.6 -6.6) (end 17.6 -8.85) (width 1.0) (layer "B.Cu") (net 20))
 (segment (start 17.6 -8.85) (end 15.6 -10.85) (width 1.0) (layer "B.Cu") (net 20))
 (segment (start 15.6 -10.85) (end 15.6 -11.6) (width 1.0) (layer "B.Cu") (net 20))
 (segment (start -9.65 -5.6) (end -12.4 -5.6) (width 0.8) (layer "B.Cu") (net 22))
 (segment (start 19.1 -1.1) (end 19.1 -0.35) (width 1.0) (layer "B.Cu") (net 6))
 (segment (start 19.1 -0.35) (end 16.1 2.65) (width 1.0) (layer "B.Cu") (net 6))
 (segment (start 16.1 2.65) (end 16.1 3.4) (width 1.0) (layer "B.Cu") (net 6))
 (segment (start 16.1 3.4) (end 16.1 3.9) (width 1.0) (layer "B.Cu") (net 6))
 (segment (start 16.1 3.9) (end 14.6 5.4) (width 1.0) (layer "B.Cu") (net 6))
 (segment (start 14.6 5.4) (end 14.1 5.4) (width 1.0) (layer "B.Cu") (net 6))
 (segment (start 14.1 5.4) (end 12.85 6.65) (width 1.0) (layer "B.Cu") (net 6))
 (segment (start 12.85 6.65) (end 12.85 7.4) (width 1.0) (layer "B.Cu") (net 6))
 (segment (start 12.85 7.4) (end 9.1 7.4) (width 1.0) (layer "B.Cu") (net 6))
 (segment (start -7.65 -3.6) (end -7.65 -1.85) (width 1.0) (layer "B.Cu") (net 6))
 (segment (start -7.65 -1.85) (end -7.65 -0.6) (width 1.0) (layer "F.Cu") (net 6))
 (segment (start -7.65 -1.35) (end -6.65 -1.35) (width 1.0) (layer "B.Cu") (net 6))
 (segment (start -6.65 -1.35) (end -5.15 -1.35) (width 1.0) (layer "F.Cu") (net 6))
 (segment (start -5.15 -1.35) (end -3.9 -0.1) (width 1.0) (layer "F.Cu") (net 6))
 (segment (start -3.9 -0.1) (end -3.9 1.9) (width 1.0) (layer "F.Cu") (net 6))
 (segment (start -3.9 1.9) (end -5.15 3.15) (width 1.0) (layer "F.Cu") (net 6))
 (segment (start -5.15 3.15) (end -7.15 3.15) (width 1.0) (layer "F.Cu") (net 6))
 (segment (start -7.15 3.15) (end -7.65 2.65) (width 1.0) (layer "F.Cu") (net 6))
 (segment (start -7.65 2.65) (end -7.65 2.4) (width 1.0) (layer "F.Cu") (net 6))
 (segment (start -5.15 -1.35) (end 2.1 -8.6) (width 1.0) (layer "F.Cu") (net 6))
 (segment (start 2.1 -8.6) (end 2.1 -8.85) (width 1.0) (layer "B.Cu") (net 6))
 (segment (start 2.1 -8.85) (end 2.85 -9.6) (width 1.0) (layer "B.Cu") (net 6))
 (segment (start -1.9 -12.1) (end -2.9 -12.1) (width 0.8) (layer "B.Cu") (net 11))
 (segment (start -2.9 -12.1) (end -5.4 -12.1) (width 0.8) (layer "F.Cu") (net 11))
 (segment (start -5.4 -12.1) (end -6.15 -11.35) (width 0.8) (layer "F.Cu") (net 11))
 (segment (start -6.15 -11.35) (end -10.65 -11.35) (width 0.8) (layer "F.Cu") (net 11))
 (segment (start -10.65 -11.35) (end -12.4 -13.1) (width 0.8) (layer "F.Cu") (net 11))
 (segment (start -12.4 -13.1) (end -12.4 -13.35) (width 0.8) (layer "B.Cu") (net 11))
 (segment (start 8.85 -1.1) (end 8.85 -2.1) (width 1.0) (layer "B.Cu") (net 21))
 (segment (start 8.85 -2.1) (end 8.85 -5.1) (width 1.0) (layer "F.Cu") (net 21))
 (segment (start 8.85 -5.1) (end 7.35 -6.6) (width 1.0) (layer "F.Cu") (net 21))
 (segment (start 7.35 -6.6) (end 7.35 -7.6) (width 1.0) (layer "B.Cu") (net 21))
 (segment (start 7.35 -7.6) (end 5.35 -9.6) (width 1.0) (layer "B.Cu") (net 21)))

